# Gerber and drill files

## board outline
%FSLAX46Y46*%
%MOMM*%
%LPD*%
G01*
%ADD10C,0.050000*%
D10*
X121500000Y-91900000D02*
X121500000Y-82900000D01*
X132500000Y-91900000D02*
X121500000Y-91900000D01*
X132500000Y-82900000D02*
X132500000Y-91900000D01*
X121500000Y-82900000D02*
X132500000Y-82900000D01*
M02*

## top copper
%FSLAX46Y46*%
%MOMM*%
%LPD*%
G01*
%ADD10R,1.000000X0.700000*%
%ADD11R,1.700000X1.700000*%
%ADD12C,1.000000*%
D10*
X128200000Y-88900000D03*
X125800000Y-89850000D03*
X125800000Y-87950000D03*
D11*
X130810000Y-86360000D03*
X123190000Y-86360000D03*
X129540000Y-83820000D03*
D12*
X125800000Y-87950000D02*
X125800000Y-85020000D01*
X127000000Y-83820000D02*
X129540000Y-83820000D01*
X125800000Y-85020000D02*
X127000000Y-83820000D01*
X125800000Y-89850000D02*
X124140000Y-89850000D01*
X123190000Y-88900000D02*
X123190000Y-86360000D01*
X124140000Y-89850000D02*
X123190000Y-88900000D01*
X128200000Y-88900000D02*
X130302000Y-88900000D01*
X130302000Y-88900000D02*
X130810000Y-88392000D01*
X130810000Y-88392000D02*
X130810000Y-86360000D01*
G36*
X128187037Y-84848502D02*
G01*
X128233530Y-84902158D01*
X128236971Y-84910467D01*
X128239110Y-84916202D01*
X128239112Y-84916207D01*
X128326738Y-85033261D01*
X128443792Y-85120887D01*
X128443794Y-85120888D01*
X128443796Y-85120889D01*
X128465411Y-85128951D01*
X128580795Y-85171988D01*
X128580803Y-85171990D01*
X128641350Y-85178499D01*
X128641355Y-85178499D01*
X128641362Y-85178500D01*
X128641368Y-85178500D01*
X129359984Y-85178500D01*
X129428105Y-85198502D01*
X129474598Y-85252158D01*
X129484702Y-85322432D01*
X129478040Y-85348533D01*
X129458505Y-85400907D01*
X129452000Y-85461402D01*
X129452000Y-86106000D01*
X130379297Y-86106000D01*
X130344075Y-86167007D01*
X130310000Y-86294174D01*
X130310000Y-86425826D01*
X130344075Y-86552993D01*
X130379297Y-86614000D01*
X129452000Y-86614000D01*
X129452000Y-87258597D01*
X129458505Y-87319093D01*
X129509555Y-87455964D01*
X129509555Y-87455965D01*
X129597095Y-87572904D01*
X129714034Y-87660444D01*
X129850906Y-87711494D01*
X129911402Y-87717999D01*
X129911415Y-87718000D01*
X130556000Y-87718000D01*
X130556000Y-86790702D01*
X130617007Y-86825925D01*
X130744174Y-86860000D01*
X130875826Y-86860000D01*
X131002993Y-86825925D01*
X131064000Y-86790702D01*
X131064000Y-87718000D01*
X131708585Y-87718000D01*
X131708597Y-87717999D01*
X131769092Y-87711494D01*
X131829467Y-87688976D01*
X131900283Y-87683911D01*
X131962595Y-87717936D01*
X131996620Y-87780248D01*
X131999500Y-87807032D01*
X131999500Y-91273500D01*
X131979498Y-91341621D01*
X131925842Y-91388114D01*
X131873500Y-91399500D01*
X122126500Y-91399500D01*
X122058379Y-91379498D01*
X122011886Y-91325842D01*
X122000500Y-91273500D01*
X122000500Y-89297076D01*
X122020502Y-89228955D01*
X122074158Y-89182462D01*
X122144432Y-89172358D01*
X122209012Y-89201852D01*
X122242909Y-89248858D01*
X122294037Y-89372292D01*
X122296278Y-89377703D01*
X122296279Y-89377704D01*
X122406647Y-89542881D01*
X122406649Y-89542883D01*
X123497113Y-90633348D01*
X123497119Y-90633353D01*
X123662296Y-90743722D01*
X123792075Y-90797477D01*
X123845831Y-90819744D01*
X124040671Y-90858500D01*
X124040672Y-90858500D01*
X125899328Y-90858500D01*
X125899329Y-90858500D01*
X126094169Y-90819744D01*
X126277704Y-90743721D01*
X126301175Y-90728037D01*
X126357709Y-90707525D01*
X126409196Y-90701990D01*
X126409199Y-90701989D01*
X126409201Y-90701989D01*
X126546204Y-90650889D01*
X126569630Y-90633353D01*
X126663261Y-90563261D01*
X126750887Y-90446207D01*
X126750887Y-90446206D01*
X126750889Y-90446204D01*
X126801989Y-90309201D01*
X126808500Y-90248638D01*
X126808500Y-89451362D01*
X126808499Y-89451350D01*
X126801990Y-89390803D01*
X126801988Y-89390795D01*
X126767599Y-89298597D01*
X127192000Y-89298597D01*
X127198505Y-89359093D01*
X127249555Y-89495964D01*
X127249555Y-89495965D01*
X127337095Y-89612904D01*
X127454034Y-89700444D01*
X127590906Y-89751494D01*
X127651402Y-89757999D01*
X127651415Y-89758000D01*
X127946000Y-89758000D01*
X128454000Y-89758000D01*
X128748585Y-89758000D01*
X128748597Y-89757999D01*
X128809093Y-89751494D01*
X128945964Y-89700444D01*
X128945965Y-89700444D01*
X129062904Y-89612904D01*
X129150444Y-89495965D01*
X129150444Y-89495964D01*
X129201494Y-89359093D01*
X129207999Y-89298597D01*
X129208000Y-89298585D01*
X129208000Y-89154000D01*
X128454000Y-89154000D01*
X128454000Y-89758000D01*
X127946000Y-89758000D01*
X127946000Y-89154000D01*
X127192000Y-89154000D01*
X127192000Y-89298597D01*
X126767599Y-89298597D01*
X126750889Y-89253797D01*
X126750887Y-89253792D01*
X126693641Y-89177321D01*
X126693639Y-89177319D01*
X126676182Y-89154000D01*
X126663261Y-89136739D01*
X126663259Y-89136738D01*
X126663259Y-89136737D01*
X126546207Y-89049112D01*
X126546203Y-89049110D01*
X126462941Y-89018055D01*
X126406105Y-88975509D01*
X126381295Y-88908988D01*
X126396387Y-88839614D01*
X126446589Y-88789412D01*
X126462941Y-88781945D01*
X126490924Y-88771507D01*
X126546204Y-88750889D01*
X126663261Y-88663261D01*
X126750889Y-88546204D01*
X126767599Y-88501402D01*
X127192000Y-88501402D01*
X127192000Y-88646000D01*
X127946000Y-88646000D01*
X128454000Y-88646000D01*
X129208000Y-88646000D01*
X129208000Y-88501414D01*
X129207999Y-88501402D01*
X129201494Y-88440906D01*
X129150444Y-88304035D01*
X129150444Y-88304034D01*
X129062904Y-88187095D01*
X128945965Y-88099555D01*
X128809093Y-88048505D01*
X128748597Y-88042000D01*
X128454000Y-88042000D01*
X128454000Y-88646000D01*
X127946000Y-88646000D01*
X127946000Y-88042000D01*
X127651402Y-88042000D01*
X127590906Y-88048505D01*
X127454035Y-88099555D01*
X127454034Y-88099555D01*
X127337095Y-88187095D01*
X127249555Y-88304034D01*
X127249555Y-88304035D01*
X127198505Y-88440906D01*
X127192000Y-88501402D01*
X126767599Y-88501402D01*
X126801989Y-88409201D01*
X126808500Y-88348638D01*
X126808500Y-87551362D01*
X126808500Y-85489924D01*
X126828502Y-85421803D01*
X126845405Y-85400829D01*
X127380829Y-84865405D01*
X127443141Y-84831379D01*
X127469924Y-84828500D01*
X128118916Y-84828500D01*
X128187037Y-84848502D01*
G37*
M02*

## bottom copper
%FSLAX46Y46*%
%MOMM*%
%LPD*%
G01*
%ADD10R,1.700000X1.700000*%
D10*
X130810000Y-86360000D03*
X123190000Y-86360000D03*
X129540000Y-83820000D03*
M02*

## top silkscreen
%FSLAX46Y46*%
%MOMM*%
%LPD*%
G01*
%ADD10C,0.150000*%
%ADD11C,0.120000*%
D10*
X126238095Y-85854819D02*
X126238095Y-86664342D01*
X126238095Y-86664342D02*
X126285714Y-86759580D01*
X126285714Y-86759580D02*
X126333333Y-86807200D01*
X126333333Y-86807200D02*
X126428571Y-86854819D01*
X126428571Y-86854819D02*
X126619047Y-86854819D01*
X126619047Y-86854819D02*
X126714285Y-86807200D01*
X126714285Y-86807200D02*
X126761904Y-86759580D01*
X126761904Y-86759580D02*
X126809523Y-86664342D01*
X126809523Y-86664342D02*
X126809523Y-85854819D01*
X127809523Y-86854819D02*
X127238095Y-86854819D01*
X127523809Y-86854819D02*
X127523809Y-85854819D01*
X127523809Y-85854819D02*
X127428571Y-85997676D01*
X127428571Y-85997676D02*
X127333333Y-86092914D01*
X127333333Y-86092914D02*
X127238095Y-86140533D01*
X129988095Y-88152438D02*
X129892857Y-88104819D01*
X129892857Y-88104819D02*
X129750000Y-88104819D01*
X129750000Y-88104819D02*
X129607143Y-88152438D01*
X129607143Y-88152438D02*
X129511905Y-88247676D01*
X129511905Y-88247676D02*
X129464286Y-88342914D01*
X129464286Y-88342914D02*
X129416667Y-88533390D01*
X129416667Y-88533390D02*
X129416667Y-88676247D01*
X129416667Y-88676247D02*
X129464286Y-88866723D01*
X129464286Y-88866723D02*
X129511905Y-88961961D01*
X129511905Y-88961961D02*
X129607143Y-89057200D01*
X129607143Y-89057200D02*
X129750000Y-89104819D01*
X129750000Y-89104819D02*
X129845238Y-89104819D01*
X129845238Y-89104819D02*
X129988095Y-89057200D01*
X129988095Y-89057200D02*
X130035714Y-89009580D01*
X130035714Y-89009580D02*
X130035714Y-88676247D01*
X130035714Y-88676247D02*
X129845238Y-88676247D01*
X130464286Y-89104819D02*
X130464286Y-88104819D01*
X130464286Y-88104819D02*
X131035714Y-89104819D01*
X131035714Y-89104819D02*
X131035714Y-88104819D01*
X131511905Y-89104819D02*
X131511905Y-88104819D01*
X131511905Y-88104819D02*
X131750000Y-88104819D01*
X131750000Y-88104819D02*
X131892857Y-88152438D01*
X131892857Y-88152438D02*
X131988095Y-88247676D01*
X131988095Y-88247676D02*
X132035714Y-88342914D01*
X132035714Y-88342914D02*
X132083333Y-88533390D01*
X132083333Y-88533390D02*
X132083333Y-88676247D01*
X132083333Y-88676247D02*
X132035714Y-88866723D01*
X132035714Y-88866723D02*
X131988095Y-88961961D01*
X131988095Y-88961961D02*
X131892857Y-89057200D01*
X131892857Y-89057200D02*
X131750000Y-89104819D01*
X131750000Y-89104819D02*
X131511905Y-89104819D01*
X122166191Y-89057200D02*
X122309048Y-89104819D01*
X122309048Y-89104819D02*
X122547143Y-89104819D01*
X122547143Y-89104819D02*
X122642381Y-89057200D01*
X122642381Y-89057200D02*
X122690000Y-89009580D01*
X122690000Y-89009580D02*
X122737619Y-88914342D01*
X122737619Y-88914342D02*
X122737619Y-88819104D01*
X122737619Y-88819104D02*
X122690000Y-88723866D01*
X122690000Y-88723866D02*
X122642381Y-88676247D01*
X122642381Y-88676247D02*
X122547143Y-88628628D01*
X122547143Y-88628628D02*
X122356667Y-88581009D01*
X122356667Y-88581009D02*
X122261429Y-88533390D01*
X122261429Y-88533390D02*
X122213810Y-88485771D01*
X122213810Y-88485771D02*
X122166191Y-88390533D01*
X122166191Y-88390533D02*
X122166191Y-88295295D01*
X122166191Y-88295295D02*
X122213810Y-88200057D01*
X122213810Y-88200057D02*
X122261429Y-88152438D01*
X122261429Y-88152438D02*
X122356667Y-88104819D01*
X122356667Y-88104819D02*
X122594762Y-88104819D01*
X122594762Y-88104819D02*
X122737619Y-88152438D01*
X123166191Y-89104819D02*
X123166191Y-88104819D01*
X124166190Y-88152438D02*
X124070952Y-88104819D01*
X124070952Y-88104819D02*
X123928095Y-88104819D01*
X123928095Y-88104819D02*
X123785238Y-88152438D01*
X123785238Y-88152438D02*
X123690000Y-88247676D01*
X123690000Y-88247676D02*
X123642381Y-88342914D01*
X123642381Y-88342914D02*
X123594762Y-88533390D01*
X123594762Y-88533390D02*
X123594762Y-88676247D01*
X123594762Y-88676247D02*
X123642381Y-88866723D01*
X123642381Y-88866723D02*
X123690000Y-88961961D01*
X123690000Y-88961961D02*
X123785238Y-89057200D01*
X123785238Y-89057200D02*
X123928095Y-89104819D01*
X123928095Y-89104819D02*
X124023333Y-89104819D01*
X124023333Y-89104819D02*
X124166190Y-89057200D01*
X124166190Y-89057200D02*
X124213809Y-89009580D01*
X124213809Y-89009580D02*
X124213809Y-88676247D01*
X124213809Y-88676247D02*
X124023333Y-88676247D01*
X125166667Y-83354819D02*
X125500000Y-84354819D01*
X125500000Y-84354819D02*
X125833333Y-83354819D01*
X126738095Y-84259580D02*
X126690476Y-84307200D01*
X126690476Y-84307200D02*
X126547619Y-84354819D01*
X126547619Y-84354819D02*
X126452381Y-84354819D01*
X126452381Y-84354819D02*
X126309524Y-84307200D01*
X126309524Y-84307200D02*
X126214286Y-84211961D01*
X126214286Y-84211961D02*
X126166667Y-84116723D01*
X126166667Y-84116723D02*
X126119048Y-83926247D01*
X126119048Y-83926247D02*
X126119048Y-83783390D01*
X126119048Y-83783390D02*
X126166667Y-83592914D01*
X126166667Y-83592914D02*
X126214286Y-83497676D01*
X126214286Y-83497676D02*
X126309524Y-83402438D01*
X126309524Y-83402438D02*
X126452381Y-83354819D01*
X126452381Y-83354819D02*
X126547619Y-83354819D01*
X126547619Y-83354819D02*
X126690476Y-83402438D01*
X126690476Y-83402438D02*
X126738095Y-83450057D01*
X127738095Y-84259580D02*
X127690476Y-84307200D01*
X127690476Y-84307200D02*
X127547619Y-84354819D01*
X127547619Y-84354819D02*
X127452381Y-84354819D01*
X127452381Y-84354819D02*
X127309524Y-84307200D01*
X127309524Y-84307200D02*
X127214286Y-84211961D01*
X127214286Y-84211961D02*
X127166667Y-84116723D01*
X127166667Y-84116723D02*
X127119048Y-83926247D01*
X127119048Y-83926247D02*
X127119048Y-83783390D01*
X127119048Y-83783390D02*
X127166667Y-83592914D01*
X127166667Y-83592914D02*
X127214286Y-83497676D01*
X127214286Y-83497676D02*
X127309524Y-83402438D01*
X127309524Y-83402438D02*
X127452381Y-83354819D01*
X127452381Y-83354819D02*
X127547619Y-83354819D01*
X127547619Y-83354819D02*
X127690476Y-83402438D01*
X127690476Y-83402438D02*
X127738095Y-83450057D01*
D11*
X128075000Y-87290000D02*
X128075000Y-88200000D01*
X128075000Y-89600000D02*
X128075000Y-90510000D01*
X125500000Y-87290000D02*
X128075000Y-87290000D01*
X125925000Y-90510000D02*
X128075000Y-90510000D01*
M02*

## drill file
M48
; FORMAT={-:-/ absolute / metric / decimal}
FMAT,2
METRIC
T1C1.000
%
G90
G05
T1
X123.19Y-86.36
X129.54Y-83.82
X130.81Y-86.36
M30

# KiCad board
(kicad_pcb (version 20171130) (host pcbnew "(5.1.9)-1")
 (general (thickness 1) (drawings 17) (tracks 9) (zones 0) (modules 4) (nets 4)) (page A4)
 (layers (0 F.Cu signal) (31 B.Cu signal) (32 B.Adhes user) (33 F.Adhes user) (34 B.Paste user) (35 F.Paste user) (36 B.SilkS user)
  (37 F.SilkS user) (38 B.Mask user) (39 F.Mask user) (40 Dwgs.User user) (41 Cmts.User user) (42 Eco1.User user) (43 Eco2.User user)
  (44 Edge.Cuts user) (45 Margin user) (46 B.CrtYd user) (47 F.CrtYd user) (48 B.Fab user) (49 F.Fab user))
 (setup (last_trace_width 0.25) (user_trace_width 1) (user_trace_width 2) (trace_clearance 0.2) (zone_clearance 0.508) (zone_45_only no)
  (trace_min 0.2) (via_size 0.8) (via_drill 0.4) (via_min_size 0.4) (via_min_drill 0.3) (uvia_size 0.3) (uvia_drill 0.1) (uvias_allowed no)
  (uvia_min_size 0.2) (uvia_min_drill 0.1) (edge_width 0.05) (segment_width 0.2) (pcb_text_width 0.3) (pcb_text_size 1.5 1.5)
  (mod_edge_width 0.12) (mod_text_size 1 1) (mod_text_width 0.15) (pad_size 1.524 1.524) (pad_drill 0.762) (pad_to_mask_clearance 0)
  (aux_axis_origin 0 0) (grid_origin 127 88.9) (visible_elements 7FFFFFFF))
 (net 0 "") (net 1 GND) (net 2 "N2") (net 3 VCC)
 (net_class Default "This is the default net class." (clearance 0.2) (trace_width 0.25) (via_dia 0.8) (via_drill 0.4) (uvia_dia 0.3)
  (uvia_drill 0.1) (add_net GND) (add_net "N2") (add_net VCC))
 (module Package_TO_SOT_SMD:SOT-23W (layer F.Cu) (at 127 88.9)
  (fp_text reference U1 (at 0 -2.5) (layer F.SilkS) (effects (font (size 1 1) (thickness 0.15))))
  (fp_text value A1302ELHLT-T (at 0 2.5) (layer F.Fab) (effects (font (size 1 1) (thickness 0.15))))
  (fp_line (start 1.075 -1.61) (end 1.075 -0.7) (layer F.SilkS) (width 0.12))
  (fp_line (start 1.075 0.7) (end 1.075 1.61) (layer F.SilkS) (width 0.12))
  (fp_line (start -1.5 -1.61) (end 1.075 -1.61) (layer F.SilkS) (width 0.12))
  (fp_line (start -1.075 1.61) (end 1.075 1.61) (layer F.SilkS) (width 0.12))
  (pad 3 smd rect (at 1.2 0) (size 1 0.7) (layers F.Cu F.Paste F.Mask) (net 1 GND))
  (pad 2 smd rect (at -1.2 0.95) (size 1 0.7) (layers F.Cu F.Paste F.Mask) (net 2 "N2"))
  (pad 1 smd rect (at -1.2 -0.95) (size 1 0.7) (layers F.Cu F.Paste F.Mask) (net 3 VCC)))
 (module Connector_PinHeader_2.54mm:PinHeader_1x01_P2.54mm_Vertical (layer B.Cu) (at 130.81 86.36)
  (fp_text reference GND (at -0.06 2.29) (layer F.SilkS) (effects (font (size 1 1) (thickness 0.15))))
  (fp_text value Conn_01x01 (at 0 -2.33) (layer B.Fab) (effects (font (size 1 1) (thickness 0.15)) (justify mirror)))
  (pad 1 thru_hole rect (at 0 0) (size 1.7 1.7) (drill 1) (layers *.Cu *.Mask) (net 1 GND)))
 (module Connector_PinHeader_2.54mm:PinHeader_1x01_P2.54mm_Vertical (layer B.Cu) (at 123.19 86.36)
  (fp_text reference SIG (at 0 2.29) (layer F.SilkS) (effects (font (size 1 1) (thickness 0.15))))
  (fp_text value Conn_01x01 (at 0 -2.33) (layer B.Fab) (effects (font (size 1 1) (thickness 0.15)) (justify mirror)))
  (pad 1 thru_hole rect (at 0 0) (size 1.7 1.7) (drill 1) (layers *.Cu *.Mask) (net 2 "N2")))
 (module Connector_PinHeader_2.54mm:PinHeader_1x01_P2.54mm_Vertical (layer B.Cu) (at 129.54 83.82)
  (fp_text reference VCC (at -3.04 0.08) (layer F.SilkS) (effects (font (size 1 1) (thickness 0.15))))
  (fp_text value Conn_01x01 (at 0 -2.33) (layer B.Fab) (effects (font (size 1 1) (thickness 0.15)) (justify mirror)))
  (pad 1 thru_hole rect (at 0 0) (size 1.7 1.7) (drill 1) (layers *.Cu *.Mask) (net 3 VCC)))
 (gr_line (start 121.5 91.9) (end 121.5 82.9) (layer Edge.Cuts) (width 0.05))
 (gr_line (start 132.5 91.9) (end 121.5 91.9) (layer Edge.Cuts) (width 0.05))
 (gr_line (start 132.5 82.9) (end 132.5 91.9) (layer Edge.Cuts) (width 0.05))
 (gr_line (start 121.5 82.9) (end 132.5 82.9) (layer Edge.Cuts) (width 0.05))
 (segment (start 125.8 87.95) (end 125.8 85.02) (width 1) (layer F.Cu) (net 3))
 (segment (start 127 83.82) (end 129.54 83.82) (width 1) (layer F.Cu) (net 3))
 (segment (start 125.8 85.02) (end 127 83.82) (width 1) (layer F.Cu) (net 3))
 (segment (start 125.8 89.85) (end 124.14 89.85) (width 1) (layer F.Cu) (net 2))
 (segment (start 123.19 88.9) (end 123.19 86.36) (width 1) (layer F.Cu) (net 2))
 (segment (start 124.14 89.85) (end 123.19 88.9) (width 1) (layer F.Cu) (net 2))
 (segment (start 128.2 88.9) (end 130.302 88.9) (width 1) (layer F.Cu) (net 1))
 (segment (start 130.302 88.9) (end 130.81 88.392) (width 1) (layer F.Cu) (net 1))
 (segment (start 130.81 88.392) (end 130.81 86.36) (width 1) (layer F.Cu) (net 1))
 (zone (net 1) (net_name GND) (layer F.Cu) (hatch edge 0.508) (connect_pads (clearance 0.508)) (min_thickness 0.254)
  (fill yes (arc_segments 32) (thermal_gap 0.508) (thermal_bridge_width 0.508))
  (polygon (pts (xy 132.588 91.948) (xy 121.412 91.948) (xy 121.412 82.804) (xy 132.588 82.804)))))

